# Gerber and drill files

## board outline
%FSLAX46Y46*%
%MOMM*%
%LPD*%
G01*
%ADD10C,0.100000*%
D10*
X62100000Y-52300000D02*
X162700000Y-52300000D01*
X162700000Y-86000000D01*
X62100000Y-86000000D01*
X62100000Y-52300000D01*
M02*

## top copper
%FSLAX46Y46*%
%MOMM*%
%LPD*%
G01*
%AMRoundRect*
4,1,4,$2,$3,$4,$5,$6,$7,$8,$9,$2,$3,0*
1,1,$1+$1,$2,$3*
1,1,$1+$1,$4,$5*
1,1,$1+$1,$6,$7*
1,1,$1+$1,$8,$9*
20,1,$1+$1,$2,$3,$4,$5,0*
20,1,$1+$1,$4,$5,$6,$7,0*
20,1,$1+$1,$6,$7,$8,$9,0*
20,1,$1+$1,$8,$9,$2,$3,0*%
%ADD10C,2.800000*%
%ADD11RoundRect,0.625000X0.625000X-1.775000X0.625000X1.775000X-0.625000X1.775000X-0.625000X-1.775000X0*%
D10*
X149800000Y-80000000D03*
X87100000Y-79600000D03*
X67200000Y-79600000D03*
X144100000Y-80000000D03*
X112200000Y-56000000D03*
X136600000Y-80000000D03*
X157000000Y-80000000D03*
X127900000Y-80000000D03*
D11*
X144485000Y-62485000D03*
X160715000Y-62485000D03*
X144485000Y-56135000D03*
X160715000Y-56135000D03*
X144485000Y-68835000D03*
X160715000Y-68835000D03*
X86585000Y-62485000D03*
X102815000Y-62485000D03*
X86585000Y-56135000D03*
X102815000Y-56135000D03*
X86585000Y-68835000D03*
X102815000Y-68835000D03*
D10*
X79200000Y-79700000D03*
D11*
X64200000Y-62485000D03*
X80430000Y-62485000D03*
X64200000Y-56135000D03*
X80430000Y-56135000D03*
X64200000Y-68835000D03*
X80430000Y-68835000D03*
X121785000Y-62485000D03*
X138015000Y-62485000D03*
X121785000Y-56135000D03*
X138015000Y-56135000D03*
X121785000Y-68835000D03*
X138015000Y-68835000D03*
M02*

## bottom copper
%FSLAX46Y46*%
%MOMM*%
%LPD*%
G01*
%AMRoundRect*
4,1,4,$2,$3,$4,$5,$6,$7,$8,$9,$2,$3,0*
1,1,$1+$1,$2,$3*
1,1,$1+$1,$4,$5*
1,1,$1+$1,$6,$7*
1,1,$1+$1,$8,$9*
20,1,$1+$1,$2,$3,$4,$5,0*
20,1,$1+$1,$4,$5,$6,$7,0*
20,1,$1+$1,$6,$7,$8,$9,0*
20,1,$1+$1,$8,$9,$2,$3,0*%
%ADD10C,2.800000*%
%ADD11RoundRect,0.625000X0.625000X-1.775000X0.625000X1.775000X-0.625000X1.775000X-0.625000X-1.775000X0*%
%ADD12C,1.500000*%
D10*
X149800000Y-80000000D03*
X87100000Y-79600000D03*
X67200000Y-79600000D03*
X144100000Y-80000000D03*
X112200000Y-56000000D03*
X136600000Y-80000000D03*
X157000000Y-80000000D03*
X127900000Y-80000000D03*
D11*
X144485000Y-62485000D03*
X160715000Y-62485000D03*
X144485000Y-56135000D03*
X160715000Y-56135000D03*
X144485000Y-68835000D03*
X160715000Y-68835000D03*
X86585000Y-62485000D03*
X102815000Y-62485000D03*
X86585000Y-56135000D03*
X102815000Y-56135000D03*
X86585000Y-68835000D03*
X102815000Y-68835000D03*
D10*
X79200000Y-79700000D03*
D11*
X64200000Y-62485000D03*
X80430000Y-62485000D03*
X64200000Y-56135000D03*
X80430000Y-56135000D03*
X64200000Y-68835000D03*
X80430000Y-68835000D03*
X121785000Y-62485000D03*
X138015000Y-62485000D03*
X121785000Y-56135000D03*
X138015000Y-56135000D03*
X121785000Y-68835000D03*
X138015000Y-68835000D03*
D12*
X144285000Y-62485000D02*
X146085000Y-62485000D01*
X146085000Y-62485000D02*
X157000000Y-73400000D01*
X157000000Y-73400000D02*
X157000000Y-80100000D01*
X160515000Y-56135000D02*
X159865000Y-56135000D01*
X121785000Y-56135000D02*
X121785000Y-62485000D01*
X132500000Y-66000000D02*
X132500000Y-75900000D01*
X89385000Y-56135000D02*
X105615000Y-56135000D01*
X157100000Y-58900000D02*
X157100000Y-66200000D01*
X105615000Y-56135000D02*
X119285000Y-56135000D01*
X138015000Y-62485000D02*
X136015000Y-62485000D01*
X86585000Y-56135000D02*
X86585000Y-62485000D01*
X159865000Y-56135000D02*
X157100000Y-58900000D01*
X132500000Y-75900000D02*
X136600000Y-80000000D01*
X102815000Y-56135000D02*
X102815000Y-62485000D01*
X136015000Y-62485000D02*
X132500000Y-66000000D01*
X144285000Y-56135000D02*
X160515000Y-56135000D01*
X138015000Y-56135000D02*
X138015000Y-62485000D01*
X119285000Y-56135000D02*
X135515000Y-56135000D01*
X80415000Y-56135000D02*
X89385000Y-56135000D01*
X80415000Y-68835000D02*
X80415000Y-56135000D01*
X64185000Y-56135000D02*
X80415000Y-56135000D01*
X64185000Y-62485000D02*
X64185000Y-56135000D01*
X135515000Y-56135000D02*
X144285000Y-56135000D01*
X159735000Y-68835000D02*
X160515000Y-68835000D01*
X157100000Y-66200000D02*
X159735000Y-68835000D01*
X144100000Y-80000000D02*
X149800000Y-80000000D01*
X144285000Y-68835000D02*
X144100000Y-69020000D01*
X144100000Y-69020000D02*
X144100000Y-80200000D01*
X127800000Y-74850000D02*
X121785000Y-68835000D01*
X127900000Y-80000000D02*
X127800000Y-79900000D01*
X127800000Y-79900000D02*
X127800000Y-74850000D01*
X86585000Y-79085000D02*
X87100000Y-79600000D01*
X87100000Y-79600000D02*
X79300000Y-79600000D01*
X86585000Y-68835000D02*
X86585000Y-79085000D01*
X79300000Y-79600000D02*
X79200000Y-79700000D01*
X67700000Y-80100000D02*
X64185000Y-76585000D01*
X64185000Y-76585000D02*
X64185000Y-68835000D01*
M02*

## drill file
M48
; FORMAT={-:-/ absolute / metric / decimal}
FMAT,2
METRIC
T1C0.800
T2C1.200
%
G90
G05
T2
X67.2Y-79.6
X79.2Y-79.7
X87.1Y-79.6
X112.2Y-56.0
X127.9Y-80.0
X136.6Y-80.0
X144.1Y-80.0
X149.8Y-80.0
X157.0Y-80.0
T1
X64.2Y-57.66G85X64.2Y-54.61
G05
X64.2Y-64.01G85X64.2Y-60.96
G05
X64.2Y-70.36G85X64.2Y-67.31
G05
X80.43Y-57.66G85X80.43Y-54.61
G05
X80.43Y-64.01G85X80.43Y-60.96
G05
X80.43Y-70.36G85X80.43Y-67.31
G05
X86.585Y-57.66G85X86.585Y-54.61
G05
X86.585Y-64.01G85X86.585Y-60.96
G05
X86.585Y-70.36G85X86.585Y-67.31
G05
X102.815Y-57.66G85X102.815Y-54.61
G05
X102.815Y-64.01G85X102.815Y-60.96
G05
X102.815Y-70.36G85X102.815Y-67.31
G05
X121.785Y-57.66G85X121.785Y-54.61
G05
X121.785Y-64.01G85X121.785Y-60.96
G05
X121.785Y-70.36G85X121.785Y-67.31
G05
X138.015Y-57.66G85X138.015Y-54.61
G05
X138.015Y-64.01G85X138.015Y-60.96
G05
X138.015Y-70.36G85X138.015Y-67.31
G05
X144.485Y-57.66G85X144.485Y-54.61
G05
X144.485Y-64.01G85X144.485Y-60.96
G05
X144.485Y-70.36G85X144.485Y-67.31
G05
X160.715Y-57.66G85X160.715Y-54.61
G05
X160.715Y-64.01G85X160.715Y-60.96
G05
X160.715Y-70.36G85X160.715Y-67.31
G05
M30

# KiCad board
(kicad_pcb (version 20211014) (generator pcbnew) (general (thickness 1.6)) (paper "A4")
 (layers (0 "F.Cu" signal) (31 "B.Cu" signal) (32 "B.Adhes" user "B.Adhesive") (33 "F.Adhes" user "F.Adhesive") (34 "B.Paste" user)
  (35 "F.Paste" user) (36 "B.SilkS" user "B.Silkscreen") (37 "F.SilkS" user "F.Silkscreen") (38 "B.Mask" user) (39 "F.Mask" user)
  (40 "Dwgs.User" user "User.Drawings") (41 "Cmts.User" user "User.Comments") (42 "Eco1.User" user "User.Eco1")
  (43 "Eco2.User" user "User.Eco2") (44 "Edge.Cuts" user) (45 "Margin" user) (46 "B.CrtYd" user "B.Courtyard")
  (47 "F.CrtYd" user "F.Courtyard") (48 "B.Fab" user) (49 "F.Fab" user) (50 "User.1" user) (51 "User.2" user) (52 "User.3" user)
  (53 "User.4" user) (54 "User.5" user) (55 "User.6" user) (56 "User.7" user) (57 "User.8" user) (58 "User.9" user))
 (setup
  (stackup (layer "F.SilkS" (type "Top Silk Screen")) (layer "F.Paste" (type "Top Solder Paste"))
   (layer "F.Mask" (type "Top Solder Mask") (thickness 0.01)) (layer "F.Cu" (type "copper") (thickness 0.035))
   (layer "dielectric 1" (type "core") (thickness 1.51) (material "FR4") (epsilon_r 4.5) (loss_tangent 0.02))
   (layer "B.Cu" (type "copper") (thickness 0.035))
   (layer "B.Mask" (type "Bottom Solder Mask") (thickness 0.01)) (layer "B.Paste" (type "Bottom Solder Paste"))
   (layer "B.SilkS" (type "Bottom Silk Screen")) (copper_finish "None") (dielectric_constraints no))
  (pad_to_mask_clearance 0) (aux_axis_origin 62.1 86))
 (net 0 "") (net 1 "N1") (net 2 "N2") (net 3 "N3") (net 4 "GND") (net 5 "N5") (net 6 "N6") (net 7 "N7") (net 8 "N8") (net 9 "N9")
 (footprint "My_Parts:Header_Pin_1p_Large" (layer "F.Cu") (at 149.8 80)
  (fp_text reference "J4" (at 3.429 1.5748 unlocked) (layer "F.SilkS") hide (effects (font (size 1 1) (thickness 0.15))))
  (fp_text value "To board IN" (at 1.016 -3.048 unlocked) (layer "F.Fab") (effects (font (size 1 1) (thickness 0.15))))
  (pad "1" thru_hole circle (at 0 0) (size 2.8 2.8) (drill 1.2) (layers *.Cu *.Mask) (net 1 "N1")))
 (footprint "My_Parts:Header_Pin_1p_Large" (layer "F.Cu") (at 87.1 79.6)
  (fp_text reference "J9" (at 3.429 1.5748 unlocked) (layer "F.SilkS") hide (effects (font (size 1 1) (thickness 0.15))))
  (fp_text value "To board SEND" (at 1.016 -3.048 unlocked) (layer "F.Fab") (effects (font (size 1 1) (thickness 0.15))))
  (pad "1" thru_hole circle (at 0 0) (size 2.8 2.8) (drill 1.2) (layers *.Cu *.Mask) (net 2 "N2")))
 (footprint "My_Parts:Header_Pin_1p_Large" (layer "F.Cu") (at 67.2 79.6)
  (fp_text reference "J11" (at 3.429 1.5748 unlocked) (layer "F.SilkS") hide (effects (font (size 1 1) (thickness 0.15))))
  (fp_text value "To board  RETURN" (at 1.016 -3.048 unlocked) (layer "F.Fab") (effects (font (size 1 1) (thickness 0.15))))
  (pad "1" thru_hole circle (at 0 0) (size 2.8 2.8) (drill 1.2) (layers *.Cu *.Mask) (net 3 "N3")))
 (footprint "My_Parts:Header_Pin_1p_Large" (layer "F.Cu") (at 144.1 80)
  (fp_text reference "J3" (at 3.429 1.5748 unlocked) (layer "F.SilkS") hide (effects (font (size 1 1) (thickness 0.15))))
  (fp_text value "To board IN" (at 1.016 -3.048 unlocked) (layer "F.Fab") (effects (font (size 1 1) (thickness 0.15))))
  (pad "1" thru_hole circle (at 0 0) (size 2.8 2.8) (drill 1.2) (layers *.Cu *.Mask) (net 1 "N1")))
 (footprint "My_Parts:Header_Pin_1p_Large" (layer "F.Cu") (at 112.2 56)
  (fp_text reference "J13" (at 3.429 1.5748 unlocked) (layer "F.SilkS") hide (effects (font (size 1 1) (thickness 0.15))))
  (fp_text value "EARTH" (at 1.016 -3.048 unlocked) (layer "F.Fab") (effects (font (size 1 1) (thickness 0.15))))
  (pad "1" thru_hole circle (at 0 0) (size 2.8 2.8) (drill 1.2) (layers *.Cu *.Mask) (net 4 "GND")))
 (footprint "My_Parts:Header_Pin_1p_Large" (layer "F.Cu") (at 136.6 80)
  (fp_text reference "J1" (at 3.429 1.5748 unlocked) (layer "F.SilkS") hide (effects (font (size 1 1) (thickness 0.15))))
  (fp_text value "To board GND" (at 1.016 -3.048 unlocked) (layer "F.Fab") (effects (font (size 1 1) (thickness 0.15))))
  (pad "1" thru_hole circle (at 0 0) (size 2.8 2.8) (drill 1.2) (layers *.Cu *.Mask) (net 4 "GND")))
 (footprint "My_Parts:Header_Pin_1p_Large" (layer "F.Cu") (at 157 80)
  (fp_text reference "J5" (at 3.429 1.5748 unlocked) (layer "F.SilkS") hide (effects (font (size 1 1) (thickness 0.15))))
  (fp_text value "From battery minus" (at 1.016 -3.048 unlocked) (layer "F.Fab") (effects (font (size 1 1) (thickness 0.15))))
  (pad "1" thru_hole circle (at 0 0) (size 2.8 2.8) (drill 1.2) (layers *.Cu *.Mask) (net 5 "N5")))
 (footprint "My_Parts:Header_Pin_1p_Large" (layer "F.Cu") (at 127.9 80)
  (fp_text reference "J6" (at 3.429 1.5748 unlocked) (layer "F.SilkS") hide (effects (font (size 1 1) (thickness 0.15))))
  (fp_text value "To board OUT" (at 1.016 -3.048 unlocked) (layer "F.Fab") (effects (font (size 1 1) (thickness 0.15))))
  (pad "1" thru_hole circle (at 0 0) (size 2.8 2.8) (drill 1.2) (layers *.Cu *.Mask) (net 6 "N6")))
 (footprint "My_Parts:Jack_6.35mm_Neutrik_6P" (layer "F.Cu") (at 144.485 68.835 90)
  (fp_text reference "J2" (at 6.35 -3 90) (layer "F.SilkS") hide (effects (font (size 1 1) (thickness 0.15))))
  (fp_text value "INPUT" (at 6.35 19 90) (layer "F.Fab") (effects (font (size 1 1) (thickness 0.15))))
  (pad "R" thru_hole roundrect (at 6.35 0 90) (size 4.8 2.5) (drill oval 3.85 0.8) (layers *.Cu *.Mask) (roundrect_rratio 0.25) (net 5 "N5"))
  (pad "RN" thru_hole roundrect (at 6.35 16.23 90) (size 4.8 2.5) (drill oval 3.85 0.8) (layers *.Cu *.Mask) (roundrect_rratio 0.25)
   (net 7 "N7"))
  (pad "S" thru_hole roundrect (at 12.7 0 90) (size 4.8 2.5) (drill oval 3.85 0.8) (layers *.Cu *.Mask) (roundrect_rratio 0.25)
   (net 4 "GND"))
  (pad "SN" thru_hole roundrect (at 12.7 16.23 90) (size 4.8 2.5) (drill oval 3.85 0.8) (layers *.Cu *.Mask) (roundrect_rratio 0.25)
   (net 4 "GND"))
  (pad "T" thru_hole roundrect (at 0 0 90) (size 4.8 2.5) (drill oval 3.85 0.8) (layers *.Cu *.Mask) (roundrect_rratio 0.25) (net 1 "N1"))
  (pad "TN" thru_hole roundrect (at 0 16.23 90) (size 4.8 2.5) (drill oval 3.85 0.8) (layers *.Cu *.Mask) (roundrect_rratio 0.25)
   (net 4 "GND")))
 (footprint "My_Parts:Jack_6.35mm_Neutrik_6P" (layer "F.Cu") (at 86.585 68.835 90)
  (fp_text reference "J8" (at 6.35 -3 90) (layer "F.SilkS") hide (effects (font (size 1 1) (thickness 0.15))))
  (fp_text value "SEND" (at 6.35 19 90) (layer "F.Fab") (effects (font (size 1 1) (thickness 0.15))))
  (pad "R" thru_hole roundrect (at 6.35 0 90) (size 4.8 2.5) (drill oval 3.85 0.8) (layers *.Cu *.Mask) (roundrect_rratio 0.25)
   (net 4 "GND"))
  (pad "RN" thru_hole roundrect (at 6.35 16.23 90) (size 4.8 2.5) (drill oval 3.85 0.8) (layers *.Cu *.Mask) (roundrect_rratio 0.25)
   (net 4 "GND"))
  (pad "S" thru_hole roundrect (at 12.7 0 90) (size 4.8 2.5) (drill oval 3.85 0.8) (layers *.Cu *.Mask) (roundrect_rratio 0.25)
   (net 4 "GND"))
  (pad "SN" thru_hole roundrect (at 12.7 16.23 90) (size 4.8 2.5) (drill oval 3.85 0.8) (layers *.Cu *.Mask) (roundrect_rratio 0.25)
   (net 4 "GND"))
  (pad "T" thru_hole roundrect (at 0 0 90) (size 4.8 2.5) (drill oval 3.85 0.8) (layers *.Cu *.Mask) (roundrect_rratio 0.25) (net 2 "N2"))
  (pad "TN" thru_hole roundrect (at 0 16.23 90) (size 4.8 2.5) (drill oval 3.85 0.8) (layers *.Cu *.Mask) (roundrect_rratio 0.25)
   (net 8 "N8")))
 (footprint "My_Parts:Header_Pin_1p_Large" (layer "F.Cu") (at 79.2 79.7)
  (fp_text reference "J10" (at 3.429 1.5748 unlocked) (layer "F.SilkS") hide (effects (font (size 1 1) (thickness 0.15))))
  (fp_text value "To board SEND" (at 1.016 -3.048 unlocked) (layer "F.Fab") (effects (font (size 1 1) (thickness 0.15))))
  (pad "1" thru_hole circle (at 0 0) (size 2.8 2.8) (drill 1.2) (layers *.Cu *.Mask) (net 2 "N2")))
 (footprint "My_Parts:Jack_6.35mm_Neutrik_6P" (layer "F.Cu") (at 64.2 68.835 90)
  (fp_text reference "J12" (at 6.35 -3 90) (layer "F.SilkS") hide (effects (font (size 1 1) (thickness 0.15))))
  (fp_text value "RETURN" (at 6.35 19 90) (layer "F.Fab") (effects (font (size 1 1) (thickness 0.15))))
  (pad "R" thru_hole roundrect (at 6.35 0 90) (size 4.8 2.5) (drill oval 3.85 0.8) (layers *.Cu *.Mask) (roundrect_rratio 0.25)
   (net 4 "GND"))
  (pad "RN" thru_hole roundrect (at 6.35 16.23 90) (size 4.8 2.5) (drill oval 3.85 0.8) (layers *.Cu *.Mask) (roundrect_rratio 0.25)
   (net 4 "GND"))
  (pad "S" thru_hole roundrect (at 12.7 0 90) (size 4.8 2.5) (drill oval 3.85 0.8) (layers *.Cu *.Mask) (roundrect_rratio 0.25)
   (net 4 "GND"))
  (pad "SN" thru_hole roundrect (at 12.7 16.23 90) (size 4.8 2.5) (drill oval 3.85 0.8) (layers *.Cu *.Mask) (roundrect_rratio 0.25)
   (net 4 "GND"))
  (pad "T" thru_hole roundrect (at 0 0 90) (size 4.8 2.5) (drill oval 3.85 0.8) (layers *.Cu *.Mask) (roundrect_rratio 0.25) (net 3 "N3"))
  (pad "TN" thru_hole roundrect (at 0 16.23 90) (size 4.8 2.5) (drill oval 3.85 0.8) (layers *.Cu *.Mask) (roundrect_rratio 0.25)
   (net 4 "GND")))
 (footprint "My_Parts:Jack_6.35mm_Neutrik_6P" (layer "F.Cu") (at 121.785 68.835 90)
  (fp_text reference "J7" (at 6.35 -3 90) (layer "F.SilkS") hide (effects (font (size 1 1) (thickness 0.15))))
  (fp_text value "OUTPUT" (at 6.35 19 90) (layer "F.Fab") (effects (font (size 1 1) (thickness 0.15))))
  (pad "R" thru_hole roundrect (at 6.35 0 90) (size 4.8 2.5) (drill oval 3.85 0.8) (layers *.Cu *.Mask) (roundrect_rratio 0.25)
   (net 4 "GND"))
  (pad "RN" thru_hole roundrect (at 6.35 16.23 90) (size 4.8 2.5) (drill oval 3.85 0.8) (layers *.Cu *.Mask) (roundrect_rratio 0.25)
   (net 4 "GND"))
  (pad "S" thru_hole roundrect (at 12.7 0 90) (size 4.8 2.5) (drill oval 3.85 0.8) (layers *.Cu *.Mask) (roundrect_rratio 0.25)
   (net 4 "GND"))
  (pad "SN" thru_hole roundrect (at 12.7 16.23 90) (size 4.8 2.5) (drill oval 3.85 0.8) (layers *.Cu *.Mask) (roundrect_rratio 0.25)
   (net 4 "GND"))
  (pad "T" thru_hole roundrect (at 0 0 90) (size 4.8 2.5) (drill oval 3.85 0.8) (layers *.Cu *.Mask) (roundrect_rratio 0.25) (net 6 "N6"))
  (pad "TN" thru_hole roundrect (at 0 16.23 90) (size 4.8 2.5) (drill oval 3.85 0.8) (layers *.Cu *.Mask) (roundrect_rratio 0.25)
   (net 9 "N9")))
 (gr_rect (start 62.1 52.3) (end 162.7 86) (layer "Edge.Cuts") (width 0.1) (fill none))
 (segment (start 144.285 62.485) (end 146.085 62.485) (width 1.5) (layer "B.Cu") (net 5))
 (segment (start 146.085 62.485) (end 157 73.4) (width 1.5) (layer "B.Cu") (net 5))
 (segment (start 157 73.4) (end 157 80.1) (width 1.5) (layer "B.Cu") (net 5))
 (segment (start 160.515 56.135) (end 159.865 56.135) (width 1.5) (layer "B.Cu") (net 4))
 (segment (start 121.785 56.135) (end 121.785 62.485) (width 1.5) (layer "B.Cu") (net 4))
 (segment (start 132.5 66) (end 132.5 75.9) (width 1.5) (layer "B.Cu") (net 4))
 (segment (start 89.385 56.135) (end 105.615 56.135) (width 1.5) (layer "B.Cu") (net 4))
 (segment (start 157.1 58.9) (end 157.1 66.2) (width 1.5) (layer "B.Cu") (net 4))
 (segment (start 105.615 56.135) (end 119.285 56.135) (width 1.5) (layer "B.Cu") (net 4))
 (segment (start 138.015 62.485) (end 136.015 62.485) (width 1.5) (layer "B.Cu") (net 4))
 (segment (start 86.585 56.135) (end 86.585 62.485) (width 1.5) (layer "B.Cu") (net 4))
 (segment (start 159.865 56.135) (end 157.1 58.9) (width 1.5) (layer "B.Cu") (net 4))
 (segment (start 132.5 75.9) (end 136.6 80) (width 1.5) (layer "B.Cu") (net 4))
 (segment (start 102.815 56.135) (end 102.815 62.485) (width 1.5) (layer "B.Cu") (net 4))
 (segment (start 136.015 62.485) (end 132.5 66) (width 1.5) (layer "B.Cu") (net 4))
 (segment (start 144.285 56.135) (end 160.515 56.135) (width 1.5) (layer "B.Cu") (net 4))
 (segment (start 138.015 56.135) (end 138.015 62.485) (width 1.5) (layer "B.Cu") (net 4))
 (segment (start 119.285 56.135) (end 135.515 56.135) (width 1.5) (layer "B.Cu") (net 4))
 (segment (start 80.415 56.135) (end 89.385 56.135) (width 1.5) (layer "B.Cu") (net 4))
 (segment (start 80.415 68.835) (end 80.415 56.135) (width 1.5) (layer "B.Cu") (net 4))
 (segment (start 64.185 56.135) (end 80.415 56.135) (width 1.5) (layer "B.Cu") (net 4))
 (segment (start 64.185 62.485) (end 64.185 56.135) (width 1.5) (layer "B.Cu") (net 4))
 (segment (start 135.515 56.135) (end 144.285 56.135) (width 1.5) (layer "B.Cu") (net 4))
 (segment (start 159.735 68.835) (end 160.515 68.835) (width 1.5) (layer "B.Cu") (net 4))
 (segment (start 157.1 66.2) (end 159.735 68.835) (width 1.5) (layer "B.Cu") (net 4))
 (segment (start 144.1 80) (end 149.8 80) (width 1.5) (layer "B.Cu") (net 1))
 (segment (start 144.285 68.835) (end 144.1 69.02) (width 1.5) (layer "B.Cu") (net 1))
 (segment (start 144.1 69.02) (end 144.1 80.2) (width 1.5) (layer "B.Cu") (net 1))
 (segment (start 127.8 74.85) (end 121.785 68.835) (width 1.5) (layer "B.Cu") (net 6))
 (segment (start 127.9 80) (end 127.8 79.9) (width 1.5) (layer "B.Cu") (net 6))
 (segment (start 127.8 79.9) (end 127.8 74.85) (width 1.5) (layer "B.Cu") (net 6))
 (segment (start 86.585 79.085) (end 87.1 79.6) (width 1.5) (layer "B.Cu") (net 2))
 (segment (start 87.1 79.6) (end 79.3 79.6) (width 1.5) (layer "B.Cu") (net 2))
 (segment (start 86.585 68.835) (end 86.585 79.085) (width 1.5) (layer "B.Cu") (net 2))
 (segment (start 79.3 79.6) (end 79.2 79.7) (width 1.5) (layer "B.Cu") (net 2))
 (segment (start 67.7 80.1) (end 64.185 76.585) (width 1.5) (layer "B.Cu") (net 3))
 (segment (start 64.185 76.585) (end 64.185 68.835) (width 1.5) (layer "B.Cu") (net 3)))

